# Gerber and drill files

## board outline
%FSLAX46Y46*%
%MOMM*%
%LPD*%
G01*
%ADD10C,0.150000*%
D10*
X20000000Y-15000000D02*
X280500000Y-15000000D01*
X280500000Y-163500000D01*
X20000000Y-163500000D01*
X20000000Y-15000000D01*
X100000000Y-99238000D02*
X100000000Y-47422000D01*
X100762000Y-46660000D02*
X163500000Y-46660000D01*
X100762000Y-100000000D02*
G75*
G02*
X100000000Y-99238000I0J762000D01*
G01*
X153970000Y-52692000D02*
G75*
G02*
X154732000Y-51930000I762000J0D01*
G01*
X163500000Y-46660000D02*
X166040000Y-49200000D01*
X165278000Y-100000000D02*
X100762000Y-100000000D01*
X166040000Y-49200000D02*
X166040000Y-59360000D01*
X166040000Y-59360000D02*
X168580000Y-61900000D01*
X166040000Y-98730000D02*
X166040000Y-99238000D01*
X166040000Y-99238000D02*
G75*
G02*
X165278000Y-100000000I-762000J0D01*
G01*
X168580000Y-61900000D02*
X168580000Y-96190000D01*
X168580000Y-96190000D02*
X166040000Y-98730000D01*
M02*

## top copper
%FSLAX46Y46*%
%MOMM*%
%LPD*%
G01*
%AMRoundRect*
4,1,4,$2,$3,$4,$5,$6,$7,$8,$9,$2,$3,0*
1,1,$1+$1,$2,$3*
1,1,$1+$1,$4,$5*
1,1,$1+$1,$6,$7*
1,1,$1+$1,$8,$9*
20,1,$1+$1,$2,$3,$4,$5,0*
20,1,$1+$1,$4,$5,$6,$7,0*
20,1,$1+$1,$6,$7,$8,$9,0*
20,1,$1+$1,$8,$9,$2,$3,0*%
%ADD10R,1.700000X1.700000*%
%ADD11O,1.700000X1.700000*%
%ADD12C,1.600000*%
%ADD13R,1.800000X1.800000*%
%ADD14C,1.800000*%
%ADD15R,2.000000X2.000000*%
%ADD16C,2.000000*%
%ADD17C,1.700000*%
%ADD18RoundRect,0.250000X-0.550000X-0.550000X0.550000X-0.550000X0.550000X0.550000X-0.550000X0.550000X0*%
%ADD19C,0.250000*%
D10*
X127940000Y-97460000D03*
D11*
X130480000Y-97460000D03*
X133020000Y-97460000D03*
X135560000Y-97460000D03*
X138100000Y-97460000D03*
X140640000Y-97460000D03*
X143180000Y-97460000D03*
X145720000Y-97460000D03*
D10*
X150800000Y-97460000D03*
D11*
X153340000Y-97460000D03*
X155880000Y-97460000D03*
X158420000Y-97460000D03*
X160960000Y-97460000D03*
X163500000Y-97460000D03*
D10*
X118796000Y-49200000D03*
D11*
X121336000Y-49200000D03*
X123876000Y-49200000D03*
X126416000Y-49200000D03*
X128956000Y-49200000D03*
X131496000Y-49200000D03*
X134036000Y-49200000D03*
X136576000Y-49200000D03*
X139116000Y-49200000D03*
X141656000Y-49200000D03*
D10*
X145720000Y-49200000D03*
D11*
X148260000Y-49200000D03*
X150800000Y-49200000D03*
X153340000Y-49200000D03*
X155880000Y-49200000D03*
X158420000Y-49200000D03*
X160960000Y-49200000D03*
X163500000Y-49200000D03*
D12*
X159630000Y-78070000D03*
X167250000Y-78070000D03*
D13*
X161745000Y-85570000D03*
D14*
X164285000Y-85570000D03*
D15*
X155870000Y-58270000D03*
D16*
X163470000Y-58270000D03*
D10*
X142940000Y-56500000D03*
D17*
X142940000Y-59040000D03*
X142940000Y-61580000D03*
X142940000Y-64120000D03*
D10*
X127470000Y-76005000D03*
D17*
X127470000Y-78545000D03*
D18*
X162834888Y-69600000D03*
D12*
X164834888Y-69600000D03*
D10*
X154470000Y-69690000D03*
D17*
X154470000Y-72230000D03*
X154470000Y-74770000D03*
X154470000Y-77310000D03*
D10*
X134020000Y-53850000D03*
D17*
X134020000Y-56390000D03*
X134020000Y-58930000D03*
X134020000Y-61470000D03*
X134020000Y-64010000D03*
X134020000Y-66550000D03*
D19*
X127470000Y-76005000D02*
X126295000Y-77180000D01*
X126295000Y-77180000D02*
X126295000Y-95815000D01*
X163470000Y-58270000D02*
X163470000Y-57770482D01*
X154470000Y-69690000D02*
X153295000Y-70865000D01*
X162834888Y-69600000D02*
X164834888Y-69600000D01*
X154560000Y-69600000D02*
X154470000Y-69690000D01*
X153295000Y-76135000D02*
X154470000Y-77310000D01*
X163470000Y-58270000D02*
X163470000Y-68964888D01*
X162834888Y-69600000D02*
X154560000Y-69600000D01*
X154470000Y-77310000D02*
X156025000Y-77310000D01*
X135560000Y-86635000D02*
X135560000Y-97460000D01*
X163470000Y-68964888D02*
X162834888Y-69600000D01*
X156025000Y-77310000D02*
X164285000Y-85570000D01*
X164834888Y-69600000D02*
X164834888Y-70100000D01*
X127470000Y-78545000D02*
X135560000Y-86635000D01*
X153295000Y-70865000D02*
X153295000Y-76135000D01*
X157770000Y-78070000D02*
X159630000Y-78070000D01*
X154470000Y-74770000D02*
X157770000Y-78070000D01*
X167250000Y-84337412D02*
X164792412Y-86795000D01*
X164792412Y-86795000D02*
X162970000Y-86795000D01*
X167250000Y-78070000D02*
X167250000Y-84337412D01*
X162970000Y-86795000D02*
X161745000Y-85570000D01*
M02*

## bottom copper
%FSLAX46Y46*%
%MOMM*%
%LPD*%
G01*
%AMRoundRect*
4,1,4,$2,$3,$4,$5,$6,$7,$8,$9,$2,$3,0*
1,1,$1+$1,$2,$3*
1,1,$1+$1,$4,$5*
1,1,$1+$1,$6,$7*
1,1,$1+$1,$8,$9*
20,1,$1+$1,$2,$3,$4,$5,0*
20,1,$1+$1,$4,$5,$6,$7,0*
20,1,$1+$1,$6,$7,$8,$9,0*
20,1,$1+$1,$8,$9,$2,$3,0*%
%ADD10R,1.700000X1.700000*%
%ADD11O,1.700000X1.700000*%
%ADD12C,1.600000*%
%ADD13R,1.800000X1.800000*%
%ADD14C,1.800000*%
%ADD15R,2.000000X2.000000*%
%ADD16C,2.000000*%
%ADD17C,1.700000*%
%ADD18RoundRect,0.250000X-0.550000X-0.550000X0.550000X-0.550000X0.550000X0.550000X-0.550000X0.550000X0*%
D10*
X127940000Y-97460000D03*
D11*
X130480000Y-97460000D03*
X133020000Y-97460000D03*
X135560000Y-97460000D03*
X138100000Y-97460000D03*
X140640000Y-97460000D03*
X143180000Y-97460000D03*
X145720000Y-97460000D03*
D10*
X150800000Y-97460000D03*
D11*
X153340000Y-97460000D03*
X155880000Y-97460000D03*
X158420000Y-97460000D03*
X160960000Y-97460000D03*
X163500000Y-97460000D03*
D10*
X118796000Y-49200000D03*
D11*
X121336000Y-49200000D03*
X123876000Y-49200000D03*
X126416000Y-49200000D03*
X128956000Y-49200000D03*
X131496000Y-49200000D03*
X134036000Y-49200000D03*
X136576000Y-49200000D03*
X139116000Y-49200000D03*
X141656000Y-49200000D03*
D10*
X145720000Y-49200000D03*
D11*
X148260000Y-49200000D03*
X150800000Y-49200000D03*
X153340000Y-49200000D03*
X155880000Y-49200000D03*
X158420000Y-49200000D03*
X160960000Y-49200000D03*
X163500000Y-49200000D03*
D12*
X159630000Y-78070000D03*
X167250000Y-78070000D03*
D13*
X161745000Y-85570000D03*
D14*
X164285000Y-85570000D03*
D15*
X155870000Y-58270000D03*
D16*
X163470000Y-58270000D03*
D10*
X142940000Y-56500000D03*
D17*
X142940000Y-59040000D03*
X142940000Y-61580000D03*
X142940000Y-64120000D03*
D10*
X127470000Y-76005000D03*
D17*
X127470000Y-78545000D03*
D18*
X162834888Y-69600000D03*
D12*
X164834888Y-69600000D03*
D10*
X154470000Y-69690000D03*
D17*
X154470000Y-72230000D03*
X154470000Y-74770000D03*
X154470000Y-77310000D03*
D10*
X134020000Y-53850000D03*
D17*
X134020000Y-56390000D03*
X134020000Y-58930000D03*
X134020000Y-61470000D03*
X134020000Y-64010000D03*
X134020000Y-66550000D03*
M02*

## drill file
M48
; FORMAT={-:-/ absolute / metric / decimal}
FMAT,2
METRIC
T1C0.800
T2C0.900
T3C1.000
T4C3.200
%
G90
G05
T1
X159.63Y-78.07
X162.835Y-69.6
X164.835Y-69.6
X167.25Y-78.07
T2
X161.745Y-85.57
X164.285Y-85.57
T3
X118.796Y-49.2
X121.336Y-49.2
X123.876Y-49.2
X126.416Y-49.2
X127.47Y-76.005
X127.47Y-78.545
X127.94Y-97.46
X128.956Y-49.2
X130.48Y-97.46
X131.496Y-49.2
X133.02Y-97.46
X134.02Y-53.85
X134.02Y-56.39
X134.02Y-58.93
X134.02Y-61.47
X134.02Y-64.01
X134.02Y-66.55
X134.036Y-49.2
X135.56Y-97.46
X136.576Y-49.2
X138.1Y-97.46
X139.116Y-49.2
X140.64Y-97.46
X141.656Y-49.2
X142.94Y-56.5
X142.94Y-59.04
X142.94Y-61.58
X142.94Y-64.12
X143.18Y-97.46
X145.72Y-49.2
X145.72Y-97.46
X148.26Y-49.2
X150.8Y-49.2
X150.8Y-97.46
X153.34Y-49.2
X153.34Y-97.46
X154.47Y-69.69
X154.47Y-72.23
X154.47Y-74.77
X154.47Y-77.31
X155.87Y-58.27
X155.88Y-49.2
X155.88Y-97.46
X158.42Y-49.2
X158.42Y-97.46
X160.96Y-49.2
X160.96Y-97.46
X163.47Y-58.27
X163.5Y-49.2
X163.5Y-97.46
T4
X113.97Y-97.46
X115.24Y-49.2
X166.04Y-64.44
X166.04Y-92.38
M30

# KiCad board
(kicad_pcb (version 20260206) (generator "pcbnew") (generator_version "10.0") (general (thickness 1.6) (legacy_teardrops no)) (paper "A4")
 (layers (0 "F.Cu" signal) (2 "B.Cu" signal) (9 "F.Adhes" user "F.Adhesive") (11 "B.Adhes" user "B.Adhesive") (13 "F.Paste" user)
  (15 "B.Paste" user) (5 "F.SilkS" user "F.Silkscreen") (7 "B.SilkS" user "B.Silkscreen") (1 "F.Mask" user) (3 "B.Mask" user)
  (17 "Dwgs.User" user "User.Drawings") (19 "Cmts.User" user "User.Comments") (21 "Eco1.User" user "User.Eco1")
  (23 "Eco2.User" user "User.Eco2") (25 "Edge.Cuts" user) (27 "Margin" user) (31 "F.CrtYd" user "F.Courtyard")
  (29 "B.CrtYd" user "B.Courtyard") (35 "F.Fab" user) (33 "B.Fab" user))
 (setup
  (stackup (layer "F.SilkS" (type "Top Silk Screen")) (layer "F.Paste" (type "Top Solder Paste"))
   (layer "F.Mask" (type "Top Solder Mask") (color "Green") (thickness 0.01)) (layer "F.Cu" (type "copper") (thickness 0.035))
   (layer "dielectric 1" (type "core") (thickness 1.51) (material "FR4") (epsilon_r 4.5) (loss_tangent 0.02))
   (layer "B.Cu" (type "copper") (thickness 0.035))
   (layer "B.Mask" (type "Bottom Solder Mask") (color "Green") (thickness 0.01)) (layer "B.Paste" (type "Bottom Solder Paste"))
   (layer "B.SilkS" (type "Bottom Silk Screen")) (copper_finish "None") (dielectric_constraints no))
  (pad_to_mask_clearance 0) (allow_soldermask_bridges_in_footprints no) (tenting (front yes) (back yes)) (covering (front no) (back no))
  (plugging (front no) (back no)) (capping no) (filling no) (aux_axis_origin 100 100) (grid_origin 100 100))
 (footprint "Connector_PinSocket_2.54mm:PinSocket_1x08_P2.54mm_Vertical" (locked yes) (layer "F.Cu") (at 127.94 97.46 90)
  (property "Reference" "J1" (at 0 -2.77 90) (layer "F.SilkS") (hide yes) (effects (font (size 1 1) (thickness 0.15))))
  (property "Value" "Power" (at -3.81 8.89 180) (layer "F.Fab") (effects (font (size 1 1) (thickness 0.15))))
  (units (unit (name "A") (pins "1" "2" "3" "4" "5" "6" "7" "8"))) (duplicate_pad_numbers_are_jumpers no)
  (pad "1" thru_hole rect (at 0 0 90) (size 1.7 1.7) (drill 1) (layers "*.Cu" "*.Mask") (remove_unused_layers no) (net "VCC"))
  (pad "2" thru_hole oval (at 0 2.54 90) (size 1.7 1.7) (drill 1) (layers "*.Cu" "*.Mask") (remove_unused_layers no) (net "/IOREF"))
  (pad "3" thru_hole oval (at 0 5.08 90) (size 1.7 1.7) (drill 1) (layers "*.Cu" "*.Mask") (remove_unused_layers no) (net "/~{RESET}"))
  (pad "4" thru_hole oval (at 0 7.62 90) (size 1.7 1.7) (drill 1) (layers "*.Cu" "*.Mask") (remove_unused_layers no) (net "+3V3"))
  (pad "5" thru_hole oval (at 0 10.16 90) (size 1.7 1.7) (drill 1) (layers "*.Cu" "*.Mask") (remove_unused_layers no) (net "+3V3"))
  (pad "6" thru_hole oval (at 0 12.7 90) (size 1.7 1.7) (drill 1) (layers "*.Cu" "*.Mask") (remove_unused_layers no) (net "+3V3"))
  (pad "7" thru_hole oval (at 0 15.24 90) (size 1.7 1.7) (drill 1) (layers "*.Cu" "*.Mask") (remove_unused_layers no) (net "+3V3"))
  (pad "8" thru_hole oval (at 0 17.78 90) (size 1.7 1.7) (drill 1) (layers "*.Cu" "*.Mask") (remove_unused_layers no) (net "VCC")))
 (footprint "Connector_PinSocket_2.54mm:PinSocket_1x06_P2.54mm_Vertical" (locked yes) (layer "F.Cu") (at 150.8 97.46 90)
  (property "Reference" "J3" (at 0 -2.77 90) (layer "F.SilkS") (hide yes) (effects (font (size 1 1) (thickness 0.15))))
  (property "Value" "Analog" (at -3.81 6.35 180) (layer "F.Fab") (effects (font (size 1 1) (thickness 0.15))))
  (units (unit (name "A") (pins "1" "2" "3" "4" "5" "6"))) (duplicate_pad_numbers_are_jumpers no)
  (pad "1" thru_hole rect (at 0 0 90) (size 1.7 1.7) (drill 1) (layers "*.Cu" "*.Mask") (remove_unused_layers no) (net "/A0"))
  (pad "2" thru_hole oval (at 0 2.54 90) (size 1.7 1.7) (drill 1) (layers "*.Cu" "*.Mask") (remove_unused_layers no) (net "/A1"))
  (pad "3" thru_hole oval (at 0 5.08 90) (size 1.7 1.7) (drill 1) (layers "*.Cu" "*.Mask") (remove_unused_layers no) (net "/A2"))
  (pad "4" thru_hole oval (at 0 7.62 90) (size 1.7 1.7) (drill 1) (layers "*.Cu" "*.Mask") (remove_unused_layers no) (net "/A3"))
  (pad "5" thru_hole oval (at 0 10.16 90) (size 1.7 1.7) (drill 1) (layers "*.Cu" "*.Mask") (remove_unused_layers no) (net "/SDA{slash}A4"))
  (pad "6" thru_hole oval (at 0 12.7 90) (size 1.7 1.7) (drill 1) (layers "*.Cu" "*.Mask") (remove_unused_layers no) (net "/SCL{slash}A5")))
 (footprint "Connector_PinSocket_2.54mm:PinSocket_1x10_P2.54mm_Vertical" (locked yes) (layer "F.Cu") (at 118.796 49.2 90)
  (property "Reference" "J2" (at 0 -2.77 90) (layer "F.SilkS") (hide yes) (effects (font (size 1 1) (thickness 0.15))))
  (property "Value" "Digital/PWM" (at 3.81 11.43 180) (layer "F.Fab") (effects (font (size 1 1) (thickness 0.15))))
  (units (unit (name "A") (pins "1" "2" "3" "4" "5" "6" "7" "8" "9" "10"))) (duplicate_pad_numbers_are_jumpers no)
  (pad "1" thru_hole rect (at 0 0 90) (size 1.7 1.7) (drill 1) (layers "*.Cu" "*.Mask") (remove_unused_layers no) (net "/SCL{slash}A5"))
  (pad "2" thru_hole oval (at 0 2.54 90) (size 1.7 1.7) (drill 1) (layers "*.Cu" "*.Mask") (remove_unused_layers no) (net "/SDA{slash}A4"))
  (pad "3" thru_hole oval (at 0 5.08 90) (size 1.7 1.7) (drill 1) (layers "*.Cu" "*.Mask") (remove_unused_layers no) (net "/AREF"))
  (pad "4" thru_hole oval (at 0 7.62 90) (size 1.7 1.7) (drill 1) (layers "*.Cu" "*.Mask") (remove_unused_layers no) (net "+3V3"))
  (pad "5" thru_hole oval (at 0 10.16 90) (size 1.7 1.7) (drill 1) (layers "*.Cu" "*.Mask") (remove_unused_layers no) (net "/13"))
  (pad "6" thru_hole oval (at 0 12.7 90) (size 1.7 1.7) (drill 1) (layers "*.Cu" "*.Mask") (remove_unused_layers no) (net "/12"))
  (pad "7" thru_hole oval (at 0 15.24 90) (size 1.7 1.7) (drill 1) (layers "*.Cu" "*.Mask") (remove_unused_layers no) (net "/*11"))
  (pad "8" thru_hole oval (at 0 17.78 90) (size 1.7 1.7) (drill 1) (layers "*.Cu" "*.Mask") (remove_unused_layers no) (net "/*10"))
  (pad "9" thru_hole oval (at 0 20.32 90) (size 1.7 1.7) (drill 1) (layers "*.Cu" "*.Mask") (remove_unused_layers no) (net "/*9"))
  (pad "10" thru_hole oval (at 0 22.86 90) (size 1.7 1.7) (drill 1) (layers "*.Cu" "*.Mask") (remove_unused_layers no) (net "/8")))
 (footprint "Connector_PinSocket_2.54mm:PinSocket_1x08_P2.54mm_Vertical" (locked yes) (layer "F.Cu") (at 145.72 49.2 90)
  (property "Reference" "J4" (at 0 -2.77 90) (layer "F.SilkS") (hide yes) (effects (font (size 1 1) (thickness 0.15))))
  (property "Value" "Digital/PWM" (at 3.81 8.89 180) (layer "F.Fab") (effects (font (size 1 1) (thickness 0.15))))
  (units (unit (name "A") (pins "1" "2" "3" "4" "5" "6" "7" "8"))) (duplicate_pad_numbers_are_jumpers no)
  (pad "1" thru_hole rect (at 0 0 90) (size 1.7 1.7) (drill 1) (layers "*.Cu" "*.Mask") (remove_unused_layers no) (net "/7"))
  (pad "2" thru_hole oval (at 0 2.54 90) (size 1.7 1.7) (drill 1) (layers "*.Cu" "*.Mask") (remove_unused_layers no) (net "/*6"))
  (pad "3" thru_hole oval (at 0 5.08 90) (size 1.7 1.7) (drill 1) (layers "*.Cu" "*.Mask") (remove_unused_layers no) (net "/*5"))
  (pad "4" thru_hole oval (at 0 7.62 90) (size 1.7 1.7) (drill 1) (layers "*.Cu" "*.Mask") (remove_unused_layers no) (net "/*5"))
  (pad "5" thru_hole oval (at 0 10.16 90) (size 1.7 1.7) (drill 1) (layers "*.Cu" "*.Mask") (remove_unused_layers no) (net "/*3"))
  (pad "6" thru_hole oval (at 0 12.7 90) (size 1.7 1.7) (drill 1) (layers "*.Cu" "*.Mask") (remove_unused_layers no) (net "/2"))
  (pad "7" thru_hole oval (at 0 15.24 90) (size 1.7 1.7) (drill 1) (layers "*.Cu" "*.Mask") (remove_unused_layers no) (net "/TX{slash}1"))
  (pad "8" thru_hole oval (at 0 17.78 90) (size 1.7 1.7) (drill 1) (layers "*.Cu" "*.Mask") (remove_unused_layers no) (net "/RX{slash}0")))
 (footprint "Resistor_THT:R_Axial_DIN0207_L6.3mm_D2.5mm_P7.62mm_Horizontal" (layer "F.Cu") (at 159.63 78.07)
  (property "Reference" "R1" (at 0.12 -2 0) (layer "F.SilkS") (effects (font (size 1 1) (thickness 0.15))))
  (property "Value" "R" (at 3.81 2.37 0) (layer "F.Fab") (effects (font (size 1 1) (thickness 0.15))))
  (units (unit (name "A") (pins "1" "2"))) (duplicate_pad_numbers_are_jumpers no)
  (pad "1" thru_hole circle (at 0 0) (size 1.6 1.6) (drill 0.8) (layers "*.Cu" "*.Mask") (remove_unused_layers no) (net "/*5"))
  (pad "2" thru_hole circle (at 7.62 0) (size 1.6 1.6) (drill 0.8) (layers "*.Cu" "*.Mask") (remove_unused_layers no) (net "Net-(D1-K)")))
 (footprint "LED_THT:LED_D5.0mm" (layer "F.Cu") (at 161.745 85.57)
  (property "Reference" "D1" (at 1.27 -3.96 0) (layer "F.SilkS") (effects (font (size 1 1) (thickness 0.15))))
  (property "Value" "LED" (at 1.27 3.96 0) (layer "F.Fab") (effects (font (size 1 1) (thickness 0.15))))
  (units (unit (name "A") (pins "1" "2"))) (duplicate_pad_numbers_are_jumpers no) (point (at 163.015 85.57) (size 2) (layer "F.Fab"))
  (pad "1" thru_hole rect (at 0 0) (size 1.8 1.8) (drill 0.9) (layers "*.Cu" "*.Mask") (remove_unused_layers no) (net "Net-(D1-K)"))
  (pad "2" thru_hole circle (at 2.54 0) (size 1.8 1.8) (drill 0.9) (layers "*.Cu" "*.Mask") (remove_unused_layers no) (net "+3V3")))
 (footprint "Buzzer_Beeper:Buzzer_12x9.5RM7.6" (layer "F.Cu") (at 155.87 58.27)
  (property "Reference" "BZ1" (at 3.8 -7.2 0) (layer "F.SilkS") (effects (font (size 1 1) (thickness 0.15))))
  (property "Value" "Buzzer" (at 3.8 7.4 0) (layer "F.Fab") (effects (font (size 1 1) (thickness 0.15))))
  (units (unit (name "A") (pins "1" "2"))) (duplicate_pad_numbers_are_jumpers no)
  (pad "1" thru_hole rect (at 0 0) (size 2 2) (drill 1) (layers "*.Cu" "*.Mask") (remove_unused_layers no) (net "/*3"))
  (pad "2" thru_hole circle (at 7.6 0) (size 2 2) (drill 1) (layers "*.Cu" "*.Mask") (remove_unused_layers no) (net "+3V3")))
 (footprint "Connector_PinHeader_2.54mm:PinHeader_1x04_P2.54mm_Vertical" (layer "F.Cu") (at 142.94 56.5)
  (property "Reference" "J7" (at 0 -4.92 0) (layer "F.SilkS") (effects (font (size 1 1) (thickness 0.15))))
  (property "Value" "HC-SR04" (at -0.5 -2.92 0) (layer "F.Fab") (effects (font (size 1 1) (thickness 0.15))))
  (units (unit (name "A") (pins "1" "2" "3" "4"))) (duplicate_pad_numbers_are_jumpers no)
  (pad "1" thru_hole rect (at 0 0) (size 1.7 1.7) (drill 1) (layers "*.Cu" "*.Mask") (remove_unused_layers no) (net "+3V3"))
  (pad "2" thru_hole circle (at 0 2.54) (size 1.7 1.7) (drill 1) (layers "*.Cu" "*.Mask") (remove_unused_layers no) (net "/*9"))
  (pad "3" thru_hole circle (at 0 5.08) (size 1.7 1.7) (drill 1) (layers "*.Cu" "*.Mask") (remove_unused_layers no) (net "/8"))
  (pad "4" thru_hole circle (at 0 7.62) (size 1.7 1.7) (drill 1) (layers "*.Cu" "*.Mask") (remove_unused_layers no) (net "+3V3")))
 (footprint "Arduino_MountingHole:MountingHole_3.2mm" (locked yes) (layer "F.Cu") (at 115.24 49.2)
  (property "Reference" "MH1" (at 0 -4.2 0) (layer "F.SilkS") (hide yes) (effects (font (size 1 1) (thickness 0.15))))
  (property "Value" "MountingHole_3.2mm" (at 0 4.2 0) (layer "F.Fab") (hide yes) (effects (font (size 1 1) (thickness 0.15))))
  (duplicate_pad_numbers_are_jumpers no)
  (pad "" np_thru_hole circle (at 0 0) (size 3.2 3.2) (drill 3.2) (layers "*.Cu" "*.Mask")))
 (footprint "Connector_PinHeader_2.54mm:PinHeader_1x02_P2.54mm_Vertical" (layer "F.Cu") (at 127.47 76.005)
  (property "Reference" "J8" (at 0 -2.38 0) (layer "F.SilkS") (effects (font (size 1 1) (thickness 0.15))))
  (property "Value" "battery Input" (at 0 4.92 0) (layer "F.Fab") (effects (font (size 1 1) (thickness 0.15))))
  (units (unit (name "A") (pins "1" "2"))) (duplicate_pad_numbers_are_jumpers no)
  (pad "1" thru_hole rect (at 0 0) (size 1.7 1.7) (drill 1) (layers "*.Cu" "*.Mask") (remove_unused_layers no) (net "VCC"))
  (pad "2" thru_hole circle (at 0 2.54) (size 1.7 1.7) (drill 1) (layers "*.Cu" "*.Mask") (remove_unused_layers no) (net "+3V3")))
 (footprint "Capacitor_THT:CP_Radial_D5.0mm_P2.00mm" (layer "F.Cu") (at 162.834888 69.6)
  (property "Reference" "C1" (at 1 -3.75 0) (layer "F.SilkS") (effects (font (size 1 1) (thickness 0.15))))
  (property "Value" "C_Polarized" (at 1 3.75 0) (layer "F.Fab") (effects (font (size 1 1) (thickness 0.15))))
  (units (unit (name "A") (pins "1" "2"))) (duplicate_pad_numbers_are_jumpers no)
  (pad "1" thru_hole roundrect (at 0 0) (size 1.6 1.6) (drill 0.8) (layers "*.Cu" "*.Mask") (remove_unused_layers no)
   (roundrect_rratio 0.15625) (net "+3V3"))
  (pad "2" thru_hole circle (at 2 0) (size 1.6 1.6) (drill 0.8) (layers "*.Cu" "*.Mask") (remove_unused_layers no) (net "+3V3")))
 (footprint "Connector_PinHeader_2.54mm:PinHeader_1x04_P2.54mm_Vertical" (layer "F.Cu") (at 154.47 69.69)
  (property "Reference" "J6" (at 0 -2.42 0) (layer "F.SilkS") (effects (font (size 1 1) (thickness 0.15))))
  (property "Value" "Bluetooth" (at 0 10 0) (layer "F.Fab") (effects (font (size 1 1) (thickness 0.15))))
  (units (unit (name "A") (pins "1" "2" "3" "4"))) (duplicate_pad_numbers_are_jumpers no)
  (pad "1" thru_hole rect (at 0 0) (size 1.7 1.7) (drill 1) (layers "*.Cu" "*.Mask") (remove_unused_layers no) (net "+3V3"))
  (pad "2" thru_hole circle (at 0 2.54) (size 1.7 1.7) (drill 1) (layers "*.Cu" "*.Mask") (remove_unused_layers no) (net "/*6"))
  (pad "3" thru_hole circle (at 0 5.08) (size 1.7 1.7) (drill 1) (layers "*.Cu" "*.Mask") (remove_unused_layers no) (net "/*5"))
  (pad "4" thru_hole circle (at 0 7.62) (size 1.7 1.7) (drill 1) (layers "*.Cu" "*.Mask") (remove_unused_layers no) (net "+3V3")))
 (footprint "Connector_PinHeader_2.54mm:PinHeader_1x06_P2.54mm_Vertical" (layer "F.Cu") (at 134.02 53.85)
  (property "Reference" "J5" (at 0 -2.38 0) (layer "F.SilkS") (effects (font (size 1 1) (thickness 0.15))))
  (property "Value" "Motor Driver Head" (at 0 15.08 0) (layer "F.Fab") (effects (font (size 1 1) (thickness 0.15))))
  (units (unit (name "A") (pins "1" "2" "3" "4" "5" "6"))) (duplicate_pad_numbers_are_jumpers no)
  (pad "1" thru_hole rect (at 0 0) (size 1.7 1.7) (drill 1) (layers "*.Cu" "*.Mask") (remove_unused_layers no) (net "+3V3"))
  (pad "2" thru_hole circle (at 0 2.54) (size 1.7 1.7) (drill 1) (layers "*.Cu" "*.Mask") (remove_unused_layers no) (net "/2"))
  (pad "3" thru_hole circle (at 0 5.08) (size 1.7 1.7) (drill 1) (layers "*.Cu" "*.Mask") (remove_unused_layers no) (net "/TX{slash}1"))
  (pad "4" thru_hole circle (at 0 7.62) (size 1.7 1.7) (drill 1) (layers "*.Cu" "*.Mask") (remove_unused_layers no) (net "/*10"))
  (pad "5" thru_hole circle (at 0 10.16) (size 1.7 1.7) (drill 1) (layers "*.Cu" "*.Mask") (remove_unused_layers no) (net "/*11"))
  (pad "6" thru_hole circle (at 0 12.7) (size 1.7 1.7) (drill 1) (layers "*.Cu" "*.Mask") (remove_unused_layers no) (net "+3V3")))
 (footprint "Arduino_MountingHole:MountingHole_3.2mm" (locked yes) (layer "F.Cu") (at 113.97 97.46)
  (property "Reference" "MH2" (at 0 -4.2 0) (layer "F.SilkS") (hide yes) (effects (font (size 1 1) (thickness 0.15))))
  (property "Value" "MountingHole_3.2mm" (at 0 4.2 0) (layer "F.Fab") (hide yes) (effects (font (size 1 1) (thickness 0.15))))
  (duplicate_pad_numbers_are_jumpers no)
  (pad "" np_thru_hole circle (at 0 0) (size 3.2 3.2) (drill 3.2) (layers "*.Cu" "*.Mask")))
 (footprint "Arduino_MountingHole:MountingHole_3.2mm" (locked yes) (layer "F.Cu") (at 166.04 64.44)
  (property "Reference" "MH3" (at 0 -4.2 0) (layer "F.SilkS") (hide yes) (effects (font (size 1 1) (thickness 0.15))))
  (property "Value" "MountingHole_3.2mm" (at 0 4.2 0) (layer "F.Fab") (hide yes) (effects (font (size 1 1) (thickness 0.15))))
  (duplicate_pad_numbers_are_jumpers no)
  (pad "" np_thru_hole circle (at 0 0) (size 3.2 3.2) (drill 3.2) (layers "*.Cu" "*.Mask")))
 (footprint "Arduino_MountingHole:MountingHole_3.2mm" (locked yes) (layer "F.Cu") (at 166.04 92.38)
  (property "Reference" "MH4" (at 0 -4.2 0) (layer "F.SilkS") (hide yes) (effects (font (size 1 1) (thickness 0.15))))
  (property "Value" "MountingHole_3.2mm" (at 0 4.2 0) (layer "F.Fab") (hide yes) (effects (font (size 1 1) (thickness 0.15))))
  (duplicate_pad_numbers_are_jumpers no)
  (pad "" np_thru_hole circle (at 0 0) (size 3.2 3.2) (drill 3.2) (layers "*.Cu" "*.Mask")))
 (gr_rect (start 20 15) (end 280.5 163.5) (stroke (width 0.15) (type default)) (fill no) (layer "Edge.Cuts"))
 (gr_line (start 100 99.238) (end 100 47.422) (stroke (width 0.15) (type solid)) (layer "Edge.Cuts"))
 (gr_line (start 100.762 46.66) (end 163.5 46.66) (stroke (width 0.15) (type solid)) (layer "Edge.Cuts"))
 (gr_arc (start 100.762 100) (mid 100.223185 99.776815) (end 100 99.238) (stroke (width 0.15) (type solid)) (layer "Edge.Cuts"))
 (gr_arc (start 153.97 52.692) (mid 154.193185 52.153185) (end 154.732 51.93) (stroke (width 0.15) (type solid)) (layer "Edge.Cuts"))
 (gr_line (start 163.5 46.66) (end 166.04 49.2) (stroke (width 0.15) (type solid)) (layer "Edge.Cuts"))
 (gr_line (start 165.278 100) (end 100.762 100) (stroke (width 0.15) (type solid)) (layer "Edge.Cuts"))
 (gr_line (start 166.04 49.2) (end 166.04 59.36) (stroke (width 0.15) (type solid)) (layer "Edge.Cuts"))
 (gr_line (start 166.04 59.36) (end 168.58 61.9) (stroke (width 0.15) (type solid)) (layer "Edge.Cuts"))
 (gr_line (start 166.04 98.73) (end 166.04 99.238) (stroke (width 0.15) (type solid)) (layer "Edge.Cuts"))
 (gr_arc (start 166.04 99.238) (mid 165.816815 99.776815) (end 165.278 100) (stroke (width 0.15) (type solid)) (layer "Edge.Cuts"))
 (gr_line (start 168.58 61.9) (end 168.58 96.19) (stroke (width 0.15) (type solid)) (layer "Edge.Cuts"))
 (gr_line (start 168.58 96.19) (end 166.04 98.73) (stroke (width 0.15) (type solid)) (layer "Edge.Cuts"))
 (segment (start 127.47 76.005) (end 126.295 77.18) (width 0.25) (layer "F.Cu") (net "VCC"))
 (segment (start 126.295 77.18) (end 126.295 95.815) (width 0.25) (layer "F.Cu") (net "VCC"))
 (segment (start 163.47 58.27) (end 163.47 57.770482) (width 0.25) (layer "F.Cu") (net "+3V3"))
 (segment (start 154.47 69.69) (end 153.295 70.865) (width 0.25) (layer "F.Cu") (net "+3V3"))
 (segment (start 162.834888 69.6) (end 164.834888 69.6) (width 0.25) (layer "F.Cu") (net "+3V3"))
 (segment (start 154.56 69.6) (end 154.47 69.69) (width 0.25) (layer "F.Cu") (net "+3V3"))
 (segment (start 153.295 76.135) (end 154.47 77.31) (width 0.25) (layer "F.Cu") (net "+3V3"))
 (segment (start 163.47 58.27) (end 163.47 68.964888) (width 0.25) (layer "F.Cu") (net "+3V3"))
 (segment (start 162.834888 69.6) (end 154.56 69.6) (width 0.25) (layer "F.Cu") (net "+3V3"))
 (segment (start 154.47 77.31) (end 156.025 77.31) (width 0.25) (layer "F.Cu") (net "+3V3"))
 (segment (start 135.56 86.635) (end 135.56 97.46) (width 0.25) (layer "F.Cu") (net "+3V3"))
 (segment (start 163.47 68.964888) (end 162.834888 69.6) (width 0.25) (layer "F.Cu") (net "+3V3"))
 (segment (start 156.025 77.31) (end 164.285 85.57) (width 0.25) (layer "F.Cu") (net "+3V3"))
 (segment (start 164.834888 69.6) (end 164.834888 70.1) (width 0.25) (layer "F.Cu") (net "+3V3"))
 (segment (start 127.47 78.545) (end 135.56 86.635) (width 0.25) (layer "F.Cu") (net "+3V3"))
 (segment (start 153.295 70.865) (end 153.295 76.135) (width 0.25) (layer "F.Cu") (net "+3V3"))
 (segment (start 157.77 78.07) (end 159.63 78.07) (width 0.25) (layer "F.Cu") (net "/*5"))
 (segment (start 154.47 74.77) (end 157.77 78.07) (width 0.25) (layer "F.Cu") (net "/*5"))
 (segment (start 167.25 84.337412) (end 164.792412 86.795) (width 0.25) (layer "F.Cu") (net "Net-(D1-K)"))
 (segment (start 164.792412 86.795) (end 162.97 86.795) (width 0.25) (layer "F.Cu") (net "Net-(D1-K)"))
 (segment (start 167.25 78.07) (end 167.25 84.337412) (width 0.25) (layer "F.Cu") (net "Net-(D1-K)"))
 (segment (start 162.97 86.795) (end 161.745 85.57) (width 0.25) (layer "F.Cu") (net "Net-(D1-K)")))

